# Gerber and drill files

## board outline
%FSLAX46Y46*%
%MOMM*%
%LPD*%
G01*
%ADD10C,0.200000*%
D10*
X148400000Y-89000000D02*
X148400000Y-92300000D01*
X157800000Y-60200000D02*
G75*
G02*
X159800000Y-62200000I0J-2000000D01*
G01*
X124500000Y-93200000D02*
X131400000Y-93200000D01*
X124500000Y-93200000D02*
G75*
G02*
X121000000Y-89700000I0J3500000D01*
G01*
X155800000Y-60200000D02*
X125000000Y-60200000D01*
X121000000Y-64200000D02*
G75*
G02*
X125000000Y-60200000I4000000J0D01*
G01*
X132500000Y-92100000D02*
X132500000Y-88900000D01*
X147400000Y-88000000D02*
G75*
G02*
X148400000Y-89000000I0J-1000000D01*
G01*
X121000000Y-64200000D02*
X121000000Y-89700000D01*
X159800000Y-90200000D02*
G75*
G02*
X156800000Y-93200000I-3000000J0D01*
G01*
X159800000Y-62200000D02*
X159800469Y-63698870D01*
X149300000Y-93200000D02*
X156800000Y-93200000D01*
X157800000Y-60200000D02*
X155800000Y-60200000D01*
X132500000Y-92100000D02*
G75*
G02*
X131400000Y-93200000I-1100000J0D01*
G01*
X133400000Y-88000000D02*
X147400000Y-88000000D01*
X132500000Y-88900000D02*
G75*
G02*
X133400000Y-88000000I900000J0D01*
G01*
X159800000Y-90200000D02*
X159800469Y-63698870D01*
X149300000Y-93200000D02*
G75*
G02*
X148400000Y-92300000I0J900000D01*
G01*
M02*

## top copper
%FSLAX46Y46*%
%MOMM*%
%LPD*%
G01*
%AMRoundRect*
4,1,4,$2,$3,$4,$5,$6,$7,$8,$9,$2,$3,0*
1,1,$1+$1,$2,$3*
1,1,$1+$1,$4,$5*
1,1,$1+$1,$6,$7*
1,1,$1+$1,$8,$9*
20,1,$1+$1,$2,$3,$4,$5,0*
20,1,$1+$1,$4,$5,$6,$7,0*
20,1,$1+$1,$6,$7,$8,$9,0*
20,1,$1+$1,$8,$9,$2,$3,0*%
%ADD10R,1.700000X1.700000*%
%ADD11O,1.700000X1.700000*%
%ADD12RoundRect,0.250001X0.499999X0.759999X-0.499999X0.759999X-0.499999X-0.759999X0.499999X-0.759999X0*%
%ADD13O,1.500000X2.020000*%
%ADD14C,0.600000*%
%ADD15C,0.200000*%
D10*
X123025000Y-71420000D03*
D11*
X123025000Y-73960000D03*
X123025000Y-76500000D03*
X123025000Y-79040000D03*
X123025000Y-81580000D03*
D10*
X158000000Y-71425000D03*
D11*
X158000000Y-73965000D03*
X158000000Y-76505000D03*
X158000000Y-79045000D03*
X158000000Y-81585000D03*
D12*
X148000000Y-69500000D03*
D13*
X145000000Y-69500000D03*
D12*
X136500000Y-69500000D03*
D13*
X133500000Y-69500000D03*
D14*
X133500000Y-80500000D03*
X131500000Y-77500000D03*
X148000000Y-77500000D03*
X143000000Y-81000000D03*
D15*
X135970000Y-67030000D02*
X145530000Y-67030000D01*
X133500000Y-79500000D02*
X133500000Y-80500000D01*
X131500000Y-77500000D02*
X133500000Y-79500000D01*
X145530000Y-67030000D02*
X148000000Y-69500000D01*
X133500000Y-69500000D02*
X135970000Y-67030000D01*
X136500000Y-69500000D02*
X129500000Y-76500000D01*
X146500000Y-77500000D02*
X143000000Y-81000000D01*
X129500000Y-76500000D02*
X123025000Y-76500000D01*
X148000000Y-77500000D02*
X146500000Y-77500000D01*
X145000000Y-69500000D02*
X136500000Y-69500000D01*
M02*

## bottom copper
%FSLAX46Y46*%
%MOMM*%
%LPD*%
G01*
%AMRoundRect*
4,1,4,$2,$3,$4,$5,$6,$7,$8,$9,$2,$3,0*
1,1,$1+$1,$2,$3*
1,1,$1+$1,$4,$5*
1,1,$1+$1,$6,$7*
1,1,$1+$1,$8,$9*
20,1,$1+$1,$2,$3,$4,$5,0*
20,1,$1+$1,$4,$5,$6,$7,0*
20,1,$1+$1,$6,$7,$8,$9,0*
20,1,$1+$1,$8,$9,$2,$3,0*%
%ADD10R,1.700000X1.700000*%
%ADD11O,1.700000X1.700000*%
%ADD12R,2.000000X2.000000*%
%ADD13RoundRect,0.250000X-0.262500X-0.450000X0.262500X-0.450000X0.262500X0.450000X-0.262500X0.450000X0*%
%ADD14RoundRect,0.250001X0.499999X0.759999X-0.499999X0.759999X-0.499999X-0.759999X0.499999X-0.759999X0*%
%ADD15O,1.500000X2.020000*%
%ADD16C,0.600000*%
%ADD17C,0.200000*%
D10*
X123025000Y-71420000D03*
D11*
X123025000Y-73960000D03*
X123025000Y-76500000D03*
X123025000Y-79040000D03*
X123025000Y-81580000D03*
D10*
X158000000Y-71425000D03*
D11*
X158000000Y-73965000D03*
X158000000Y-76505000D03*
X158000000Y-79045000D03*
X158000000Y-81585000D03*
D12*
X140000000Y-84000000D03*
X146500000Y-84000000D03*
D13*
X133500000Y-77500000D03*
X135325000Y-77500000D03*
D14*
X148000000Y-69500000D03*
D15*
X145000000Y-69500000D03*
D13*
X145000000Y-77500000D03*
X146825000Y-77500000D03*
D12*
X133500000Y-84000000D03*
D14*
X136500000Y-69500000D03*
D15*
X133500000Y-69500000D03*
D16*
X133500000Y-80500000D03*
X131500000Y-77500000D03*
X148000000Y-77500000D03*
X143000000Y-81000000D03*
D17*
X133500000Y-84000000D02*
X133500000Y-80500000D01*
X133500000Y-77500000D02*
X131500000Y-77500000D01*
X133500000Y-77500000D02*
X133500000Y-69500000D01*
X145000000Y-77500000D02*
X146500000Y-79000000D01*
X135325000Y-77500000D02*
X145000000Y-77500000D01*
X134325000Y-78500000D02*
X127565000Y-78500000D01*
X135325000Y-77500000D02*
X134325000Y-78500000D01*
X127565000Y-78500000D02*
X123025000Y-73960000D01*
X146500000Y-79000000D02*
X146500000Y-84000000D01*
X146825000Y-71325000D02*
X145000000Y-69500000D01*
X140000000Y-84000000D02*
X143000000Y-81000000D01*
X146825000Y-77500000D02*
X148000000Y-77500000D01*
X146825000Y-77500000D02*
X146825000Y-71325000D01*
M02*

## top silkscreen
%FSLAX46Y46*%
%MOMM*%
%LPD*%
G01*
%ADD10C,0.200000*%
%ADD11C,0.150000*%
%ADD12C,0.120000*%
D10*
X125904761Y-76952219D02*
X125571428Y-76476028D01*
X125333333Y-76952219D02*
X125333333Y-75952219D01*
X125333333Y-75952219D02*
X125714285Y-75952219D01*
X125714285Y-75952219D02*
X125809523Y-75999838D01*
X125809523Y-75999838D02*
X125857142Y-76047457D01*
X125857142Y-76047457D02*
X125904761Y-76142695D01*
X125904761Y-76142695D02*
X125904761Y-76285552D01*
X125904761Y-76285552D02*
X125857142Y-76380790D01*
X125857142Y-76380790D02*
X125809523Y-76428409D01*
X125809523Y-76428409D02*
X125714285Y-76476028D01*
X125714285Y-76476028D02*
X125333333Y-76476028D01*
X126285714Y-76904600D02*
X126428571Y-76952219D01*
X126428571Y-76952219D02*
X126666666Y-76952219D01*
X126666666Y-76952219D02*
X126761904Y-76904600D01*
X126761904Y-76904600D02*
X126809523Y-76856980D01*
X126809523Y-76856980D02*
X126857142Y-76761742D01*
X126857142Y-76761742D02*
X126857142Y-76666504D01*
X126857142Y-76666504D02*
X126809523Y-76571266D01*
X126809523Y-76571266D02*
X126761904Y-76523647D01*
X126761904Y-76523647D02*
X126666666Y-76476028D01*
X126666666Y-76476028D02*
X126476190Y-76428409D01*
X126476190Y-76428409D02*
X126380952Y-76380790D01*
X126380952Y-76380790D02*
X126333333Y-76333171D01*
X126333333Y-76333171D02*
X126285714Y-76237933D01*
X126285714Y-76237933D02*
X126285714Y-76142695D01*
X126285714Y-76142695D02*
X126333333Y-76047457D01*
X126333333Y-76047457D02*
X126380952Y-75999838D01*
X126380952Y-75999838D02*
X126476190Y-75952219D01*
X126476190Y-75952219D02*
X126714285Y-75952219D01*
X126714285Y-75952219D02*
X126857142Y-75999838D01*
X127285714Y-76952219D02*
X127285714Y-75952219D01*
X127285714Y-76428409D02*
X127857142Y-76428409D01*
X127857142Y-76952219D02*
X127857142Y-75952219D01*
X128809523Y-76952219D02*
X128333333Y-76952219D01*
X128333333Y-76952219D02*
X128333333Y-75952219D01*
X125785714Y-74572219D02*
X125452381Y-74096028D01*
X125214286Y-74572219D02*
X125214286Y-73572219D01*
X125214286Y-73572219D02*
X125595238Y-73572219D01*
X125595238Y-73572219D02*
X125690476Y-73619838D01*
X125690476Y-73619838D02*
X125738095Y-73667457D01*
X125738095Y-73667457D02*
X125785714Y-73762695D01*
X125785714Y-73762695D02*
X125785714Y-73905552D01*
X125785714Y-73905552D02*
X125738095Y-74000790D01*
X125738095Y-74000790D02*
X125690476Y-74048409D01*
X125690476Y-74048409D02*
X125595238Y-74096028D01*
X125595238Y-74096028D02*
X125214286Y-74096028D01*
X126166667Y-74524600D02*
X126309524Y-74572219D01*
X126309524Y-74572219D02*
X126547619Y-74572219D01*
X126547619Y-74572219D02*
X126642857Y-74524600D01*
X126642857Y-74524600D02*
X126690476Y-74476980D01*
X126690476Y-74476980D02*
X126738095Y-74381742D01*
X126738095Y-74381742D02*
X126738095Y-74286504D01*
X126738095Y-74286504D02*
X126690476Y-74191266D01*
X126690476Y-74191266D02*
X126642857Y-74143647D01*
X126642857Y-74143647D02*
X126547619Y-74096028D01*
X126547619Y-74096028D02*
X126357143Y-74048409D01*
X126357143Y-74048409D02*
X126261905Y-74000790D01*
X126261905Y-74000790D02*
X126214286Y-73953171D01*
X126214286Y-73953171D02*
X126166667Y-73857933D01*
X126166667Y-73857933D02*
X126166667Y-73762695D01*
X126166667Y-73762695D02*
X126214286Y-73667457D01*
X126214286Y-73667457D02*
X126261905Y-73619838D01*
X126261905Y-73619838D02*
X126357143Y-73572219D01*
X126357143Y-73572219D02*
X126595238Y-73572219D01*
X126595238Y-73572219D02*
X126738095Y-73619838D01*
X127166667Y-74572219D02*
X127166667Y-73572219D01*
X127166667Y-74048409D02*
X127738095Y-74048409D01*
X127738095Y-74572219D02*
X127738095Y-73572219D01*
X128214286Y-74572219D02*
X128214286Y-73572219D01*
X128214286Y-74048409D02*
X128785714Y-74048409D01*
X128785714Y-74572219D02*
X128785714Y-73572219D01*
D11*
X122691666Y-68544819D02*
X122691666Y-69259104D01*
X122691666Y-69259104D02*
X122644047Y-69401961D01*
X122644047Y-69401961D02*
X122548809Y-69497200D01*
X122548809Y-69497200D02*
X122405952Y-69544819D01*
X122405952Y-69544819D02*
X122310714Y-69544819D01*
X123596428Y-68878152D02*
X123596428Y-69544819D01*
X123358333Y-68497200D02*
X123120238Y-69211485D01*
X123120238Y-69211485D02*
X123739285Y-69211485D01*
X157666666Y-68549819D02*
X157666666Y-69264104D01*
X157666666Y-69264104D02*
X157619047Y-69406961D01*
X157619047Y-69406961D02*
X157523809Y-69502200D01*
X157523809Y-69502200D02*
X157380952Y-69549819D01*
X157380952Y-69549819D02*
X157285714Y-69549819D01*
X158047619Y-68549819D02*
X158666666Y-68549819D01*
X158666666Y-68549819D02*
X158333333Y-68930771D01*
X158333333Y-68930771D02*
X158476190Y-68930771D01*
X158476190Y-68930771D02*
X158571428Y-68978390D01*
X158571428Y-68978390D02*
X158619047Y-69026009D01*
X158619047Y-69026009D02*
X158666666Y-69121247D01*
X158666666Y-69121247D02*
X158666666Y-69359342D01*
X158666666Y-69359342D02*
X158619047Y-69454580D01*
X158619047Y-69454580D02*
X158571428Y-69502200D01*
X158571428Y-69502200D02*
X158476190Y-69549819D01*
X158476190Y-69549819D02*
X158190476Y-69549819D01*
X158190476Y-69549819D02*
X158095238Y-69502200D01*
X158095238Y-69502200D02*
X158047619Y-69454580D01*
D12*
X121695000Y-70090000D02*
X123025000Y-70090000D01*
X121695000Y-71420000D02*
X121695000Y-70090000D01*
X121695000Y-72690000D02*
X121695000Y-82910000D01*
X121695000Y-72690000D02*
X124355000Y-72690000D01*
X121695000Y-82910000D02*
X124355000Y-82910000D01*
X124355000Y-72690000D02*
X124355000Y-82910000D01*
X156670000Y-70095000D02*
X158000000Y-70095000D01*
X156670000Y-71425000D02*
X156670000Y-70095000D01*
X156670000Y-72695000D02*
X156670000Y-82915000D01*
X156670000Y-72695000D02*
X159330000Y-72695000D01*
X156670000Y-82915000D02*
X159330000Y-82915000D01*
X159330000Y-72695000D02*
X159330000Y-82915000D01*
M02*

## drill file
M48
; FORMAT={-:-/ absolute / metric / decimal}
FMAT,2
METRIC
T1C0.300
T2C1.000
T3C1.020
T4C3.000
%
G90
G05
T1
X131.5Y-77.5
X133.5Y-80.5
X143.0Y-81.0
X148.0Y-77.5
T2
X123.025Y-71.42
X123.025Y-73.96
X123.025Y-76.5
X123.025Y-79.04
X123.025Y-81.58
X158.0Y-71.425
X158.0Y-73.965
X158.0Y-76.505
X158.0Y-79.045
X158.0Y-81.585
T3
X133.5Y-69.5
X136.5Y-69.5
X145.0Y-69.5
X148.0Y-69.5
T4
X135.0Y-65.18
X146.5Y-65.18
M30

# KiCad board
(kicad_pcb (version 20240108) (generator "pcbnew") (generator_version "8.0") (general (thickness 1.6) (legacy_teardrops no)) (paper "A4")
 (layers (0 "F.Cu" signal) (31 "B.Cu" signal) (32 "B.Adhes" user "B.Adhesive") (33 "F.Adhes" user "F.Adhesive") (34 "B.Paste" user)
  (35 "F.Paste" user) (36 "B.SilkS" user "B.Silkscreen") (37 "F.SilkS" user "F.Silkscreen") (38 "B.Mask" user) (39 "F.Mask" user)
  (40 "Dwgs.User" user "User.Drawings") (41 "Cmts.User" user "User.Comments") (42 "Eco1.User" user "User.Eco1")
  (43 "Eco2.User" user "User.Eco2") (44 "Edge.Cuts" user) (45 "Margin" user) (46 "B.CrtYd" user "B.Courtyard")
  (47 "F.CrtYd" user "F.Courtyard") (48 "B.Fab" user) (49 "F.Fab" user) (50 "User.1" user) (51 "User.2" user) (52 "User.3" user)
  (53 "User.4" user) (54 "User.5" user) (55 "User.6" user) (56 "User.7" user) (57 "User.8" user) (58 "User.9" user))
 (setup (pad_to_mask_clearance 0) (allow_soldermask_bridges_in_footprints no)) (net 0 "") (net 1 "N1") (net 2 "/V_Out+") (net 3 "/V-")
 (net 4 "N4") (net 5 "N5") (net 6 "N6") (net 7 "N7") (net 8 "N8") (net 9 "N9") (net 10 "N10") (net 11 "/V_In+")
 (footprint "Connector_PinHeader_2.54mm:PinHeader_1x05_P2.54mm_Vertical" (layer "F.Cu") (at 123.025 71.42)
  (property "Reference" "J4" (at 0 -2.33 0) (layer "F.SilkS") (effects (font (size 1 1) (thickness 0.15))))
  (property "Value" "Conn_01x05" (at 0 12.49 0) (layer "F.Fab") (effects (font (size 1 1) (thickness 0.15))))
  (fp_line (start -1.33 -1.33) (end 0 -1.33) (stroke (width 0.12) (type solid)) (layer "F.SilkS"))
  (fp_line (start -1.33 0) (end -1.33 -1.33) (stroke (width 0.12) (type solid)) (layer "F.SilkS"))
  (fp_line (start -1.33 1.27) (end -1.33 11.49) (stroke (width 0.12) (type solid)) (layer "F.SilkS"))
  (fp_line (start -1.33 1.27) (end 1.33 1.27) (stroke (width 0.12) (type solid)) (layer "F.SilkS"))
  (fp_line (start -1.33 11.49) (end 1.33 11.49) (stroke (width 0.12) (type solid)) (layer "F.SilkS"))
  (fp_line (start 1.33 1.27) (end 1.33 11.49) (stroke (width 0.12) (type solid)) (layer "F.SilkS"))
  (pad "1" thru_hole rect (at 0 0) (size 1.7 1.7) (drill 1) (layers "*.Cu" "*.Mask") (remove_unused_layers no) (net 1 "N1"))
  (pad "2" thru_hole oval (at 0 2.54) (size 1.7 1.7) (drill 1) (layers "*.Cu" "*.Mask") (remove_unused_layers no) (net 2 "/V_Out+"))
  (pad "3" thru_hole oval (at 0 5.08) (size 1.7 1.7) (drill 1) (layers "*.Cu" "*.Mask") (remove_unused_layers no) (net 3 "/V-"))
  (pad "4" thru_hole oval (at 0 7.62) (size 1.7 1.7) (drill 1) (layers "*.Cu" "*.Mask") (remove_unused_layers no) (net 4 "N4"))
  (pad "5" thru_hole oval (at 0 10.16) (size 1.7 1.7) (drill 1) (layers "*.Cu" "*.Mask") (remove_unused_layers no) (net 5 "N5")))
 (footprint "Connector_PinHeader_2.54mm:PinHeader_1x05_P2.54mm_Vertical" (layer "F.Cu") (at 158 71.425)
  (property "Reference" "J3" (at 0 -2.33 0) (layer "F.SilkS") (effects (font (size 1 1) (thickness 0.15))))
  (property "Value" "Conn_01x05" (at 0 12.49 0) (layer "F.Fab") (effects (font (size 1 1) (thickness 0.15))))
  (fp_line (start -1.33 -1.33) (end 0 -1.33) (stroke (width 0.12) (type solid)) (layer "F.SilkS"))
  (fp_line (start -1.33 0) (end -1.33 -1.33) (stroke (width 0.12) (type solid)) (layer "F.SilkS"))
  (fp_line (start -1.33 1.27) (end -1.33 11.49) (stroke (width 0.12) (type solid)) (layer "F.SilkS"))
  (fp_line (start -1.33 1.27) (end 1.33 1.27) (stroke (width 0.12) (type solid)) (layer "F.SilkS"))
  (fp_line (start -1.33 11.49) (end 1.33 11.49) (stroke (width 0.12) (type solid)) (layer "F.SilkS"))
  (fp_line (start 1.33 1.27) (end 1.33 11.49) (stroke (width 0.12) (type solid)) (layer "F.SilkS"))
  (pad "1" thru_hole rect (at 0 0) (size 1.7 1.7) (drill 1) (layers "*.Cu" "*.Mask") (remove_unused_layers no) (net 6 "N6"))
  (pad "2" thru_hole oval (at 0 2.54) (size 1.7 1.7) (drill 1) (layers "*.Cu" "*.Mask") (remove_unused_layers no) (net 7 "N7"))
  (pad "3" thru_hole oval (at 0 5.08) (size 1.7 1.7) (drill 1) (layers "*.Cu" "*.Mask") (remove_unused_layers no) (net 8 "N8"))
  (pad "4" thru_hole oval (at 0 7.62) (size 1.7 1.7) (drill 1) (layers "*.Cu" "*.Mask") (remove_unused_layers no) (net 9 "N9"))
  (pad "5" thru_hole oval (at 0 10.16) (size 1.7 1.7) (drill 1) (layers "*.Cu" "*.Mask") (remove_unused_layers no) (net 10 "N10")))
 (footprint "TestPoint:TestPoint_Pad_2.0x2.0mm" (layer "B.Cu") (at 140 84 180)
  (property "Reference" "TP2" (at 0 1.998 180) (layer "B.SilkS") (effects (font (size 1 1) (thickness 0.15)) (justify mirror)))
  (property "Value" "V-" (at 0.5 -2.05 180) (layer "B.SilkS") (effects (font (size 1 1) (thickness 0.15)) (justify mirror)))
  (pad "1" smd rect (at 0 0 180) (size 2 2) (layers "B.Cu" "B.Mask") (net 3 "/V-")))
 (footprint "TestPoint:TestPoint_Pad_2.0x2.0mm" (layer "B.Cu") (at 146.5 84 180)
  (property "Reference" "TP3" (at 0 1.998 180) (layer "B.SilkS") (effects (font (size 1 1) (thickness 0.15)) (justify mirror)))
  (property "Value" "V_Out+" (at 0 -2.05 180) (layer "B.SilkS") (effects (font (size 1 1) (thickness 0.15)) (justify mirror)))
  (pad "1" smd rect (at 0 0 180) (size 2 2) (layers "B.Cu" "B.Mask") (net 2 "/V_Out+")))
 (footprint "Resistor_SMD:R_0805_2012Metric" (layer "B.Cu") (at 134.4125 77.5)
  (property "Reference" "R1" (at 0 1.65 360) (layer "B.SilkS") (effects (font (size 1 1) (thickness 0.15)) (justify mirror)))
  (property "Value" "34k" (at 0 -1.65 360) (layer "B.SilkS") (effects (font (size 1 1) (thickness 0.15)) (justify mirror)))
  (pad "1" smd roundrect (at -0.9125 0) (size 1.025 1.4) (layers "B.Cu" "B.Paste" "B.Mask") (roundrect_rratio 0.243902) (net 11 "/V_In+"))
  (pad "2" smd roundrect (at 0.9125 0) (size 1.025 1.4) (layers "B.Cu" "B.Paste" "B.Mask") (roundrect_rratio 0.243902) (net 2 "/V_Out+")))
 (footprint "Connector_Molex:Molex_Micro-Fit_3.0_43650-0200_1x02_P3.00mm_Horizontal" (layer "B.Cu") (at 148 69.5 180)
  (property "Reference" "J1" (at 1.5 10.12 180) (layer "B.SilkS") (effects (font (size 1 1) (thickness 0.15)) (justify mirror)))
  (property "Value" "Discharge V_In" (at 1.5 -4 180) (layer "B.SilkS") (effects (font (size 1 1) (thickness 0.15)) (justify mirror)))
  (pad "" np_thru_hole circle (at 1.5 4.32 180) (size 3 3) (drill 3) (layers "*.Cu" "*.Mask"))
  (pad "1" thru_hole roundrect (at 0 0 180) (size 1.5 2.02) (drill 1.02) (layers "*.Cu" "*.Mask") (remove_unused_layers no)
   (roundrect_rratio 0.166667) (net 11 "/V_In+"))
  (pad "2" thru_hole oval (at 3 0 180) (size 1.5 2.02) (drill 1.02) (layers "*.Cu" "*.Mask") (remove_unused_layers no) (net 3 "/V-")))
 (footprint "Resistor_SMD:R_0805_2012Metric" (layer "B.Cu") (at 145.9125 77.5)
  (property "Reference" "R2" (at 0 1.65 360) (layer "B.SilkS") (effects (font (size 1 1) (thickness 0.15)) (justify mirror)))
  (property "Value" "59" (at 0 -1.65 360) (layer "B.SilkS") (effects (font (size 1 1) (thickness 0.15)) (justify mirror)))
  (pad "1" smd roundrect (at -0.9125 0) (size 1.025 1.4) (layers "B.Cu" "B.Paste" "B.Mask") (roundrect_rratio 0.243902) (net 2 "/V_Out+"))
  (pad "2" smd roundrect (at 0.9125 0) (size 1.025 1.4) (layers "B.Cu" "B.Paste" "B.Mask") (roundrect_rratio 0.243902) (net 3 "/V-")))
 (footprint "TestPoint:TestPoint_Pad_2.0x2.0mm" (layer "B.Cu") (at 133.5 84 180)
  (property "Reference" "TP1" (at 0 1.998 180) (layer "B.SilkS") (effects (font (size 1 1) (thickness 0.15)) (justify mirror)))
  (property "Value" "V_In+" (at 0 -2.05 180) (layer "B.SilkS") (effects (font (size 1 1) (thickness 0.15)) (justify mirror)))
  (pad "1" smd rect (at 0 0 180) (size 2 2) (layers "B.Cu" "B.Mask") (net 11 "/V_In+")))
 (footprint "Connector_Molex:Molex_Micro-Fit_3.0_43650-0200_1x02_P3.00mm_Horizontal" (layer "B.Cu") (at 136.5 69.5 180)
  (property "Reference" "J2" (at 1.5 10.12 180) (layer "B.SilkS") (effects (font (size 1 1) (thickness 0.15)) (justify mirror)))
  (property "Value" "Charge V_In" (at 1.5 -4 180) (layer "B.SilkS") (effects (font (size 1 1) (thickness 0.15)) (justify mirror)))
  (pad "" np_thru_hole circle (at 1.5 4.32 180) (size 3 3) (drill 3) (layers "*.Cu" "*.Mask"))
  (pad "1" thru_hole roundrect (at 0 0 180) (size 1.5 2.02) (drill 1.02) (layers "*.Cu" "*.Mask") (remove_unused_layers no)
   (roundrect_rratio 0.166667) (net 3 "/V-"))
  (pad "2" thru_hole oval (at 3 0 180) (size 1.5 2.02) (drill 1.02) (layers "*.Cu" "*.Mask") (remove_unused_layers no) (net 11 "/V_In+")))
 (gr_line (start 148.4 89) (end 148.4 92.3) (stroke (width 0.2) (type solid)) (layer "Edge.Cuts"))
 (gr_arc (start 157.8 60.2) (mid 159.214214 60.785786) (end 159.8 62.2) (stroke (width 0.2) (type solid)) (layer "Edge.Cuts"))
 (gr_line (start 124.5 93.2) (end 131.4 93.2) (stroke (width 0.2) (type solid)) (layer "Edge.Cuts"))
 (gr_arc (start 124.5 93.2) (mid 122.025126 92.174874) (end 121 89.7) (stroke (width 0.2) (type solid)) (layer "Edge.Cuts"))
 (gr_line (start 155.8 60.2) (end 125 60.2) (stroke (width 0.2) (type solid)) (layer "Edge.Cuts"))
 (gr_arc (start 121 64.2) (mid 122.171573 61.371573) (end 125 60.2) (stroke (width 0.2) (type solid)) (layer "Edge.Cuts"))
 (gr_line (start 132.5 92.1) (end 132.5 88.9) (stroke (width 0.2) (type solid)) (layer "Edge.Cuts"))
 (gr_arc (start 147.4 88) (mid 148.107107 88.292893) (end 148.4 89) (stroke (width 0.2) (type solid)) (layer "Edge.Cuts"))
 (gr_line (start 121 64.2) (end 121 89.7) (stroke (width 0.2) (type solid)) (layer "Edge.Cuts"))
 (gr_arc (start 159.8 90.2) (mid 158.92132 92.32132) (end 156.8 93.2) (stroke (width 0.2) (type solid)) (layer "Edge.Cuts"))
 (gr_line (start 159.8 62.2) (end 159.800469 63.69887) (stroke (width 0.2) (type solid)) (layer "Edge.Cuts"))
 (gr_line (start 149.3 93.2) (end 156.8 93.2) (stroke (width 0.2) (type solid)) (layer "Edge.Cuts"))
 (gr_line (start 157.8 60.2) (end 155.8 60.2) (stroke (width 0.2) (type solid)) (layer "Edge.Cuts"))
 (gr_arc (start 132.5 92.1) (mid 132.177817 92.877817) (end 131.4 93.2) (stroke (width 0.2) (type solid)) (layer "Edge.Cuts"))
 (gr_line (start 133.4 88) (end 147.4 88) (stroke (width 0.2) (type solid)) (layer "Edge.Cuts"))
 (gr_arc (start 132.5 88.9) (mid 132.763604 88.263604) (end 133.4 88) (stroke (width 0.2) (type solid)) (layer "Edge.Cuts"))
 (gr_line (start 159.8 90.2) (end 159.800469 63.69887) (stroke (width 0.2) (type solid)) (layer "Edge.Cuts"))
 (gr_arc (start 149.3 93.2) (mid 148.663604 92.936396) (end 148.4 92.3) (stroke (width 0.2) (type solid)) (layer "Edge.Cuts"))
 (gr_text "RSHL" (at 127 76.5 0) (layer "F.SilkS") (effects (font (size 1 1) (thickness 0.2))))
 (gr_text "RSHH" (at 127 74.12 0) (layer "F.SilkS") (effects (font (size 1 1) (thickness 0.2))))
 (segment (start 135.97 67.03) (end 145.53 67.03) (width 0.2) (layer "F.Cu") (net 11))
 (segment (start 133.5 79.5) (end 133.5 80.5) (width 0.2) (layer "F.Cu") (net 11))
 (segment (start 131.5 77.5) (end 133.5 79.5) (width 0.2) (layer "F.Cu") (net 11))
 (segment (start 145.53 67.03) (end 148 69.5) (width 0.2) (layer "F.Cu") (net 11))
 (segment (start 133.5 69.5) (end 135.97 67.03) (width 0.2) (layer "F.Cu") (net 11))
 (via (at 133.5 80.5) (size 0.6) (drill 0.3) (layers "F.Cu" "B.Cu") (free yes) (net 11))
 (via (at 131.5 77.5) (size 0.6) (drill 0.3) (layers "F.Cu" "B.Cu") (free yes) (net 11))
 (segment (start 133.5 84) (end 133.5 80.5) (width 0.2) (layer "B.Cu") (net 11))
 (segment (start 133.5 77.5) (end 131.5 77.5) (width 0.2) (layer "B.Cu") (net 11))
 (segment (start 133.5 77.5) (end 133.5 69.5) (width 0.2) (layer "B.Cu") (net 11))
 (segment (start 145 77.5) (end 146.5 79) (width 0.2) (layer "B.Cu") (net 2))
 (segment (start 135.325 77.5) (end 145 77.5) (width 0.2) (layer "B.Cu") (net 2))
 (segment (start 134.325 78.5) (end 127.565 78.5) (width 0.2) (layer "B.Cu") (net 2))
 (segment (start 135.325 77.5) (end 134.325 78.5) (width 0.2) (layer "B.Cu") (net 2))
 (segment (start 127.565 78.5) (end 123.025 73.96) (width 0.2) (layer "B.Cu") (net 2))
 (segment (start 146.5 79) (end 146.5 84) (width 0.2) (layer "B.Cu") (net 2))
 (segment (start 136.5 69.5) (end 129.5 76.5) (width 0.2) (layer "F.Cu") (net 3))
 (segment (start 146.5 77.5) (end 143 81) (width 0.2) (layer "F.Cu") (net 3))
 (segment (start 129.5 76.5) (end 123.025 76.5) (width 0.2) (layer "F.Cu") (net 3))
 (segment (start 148 77.5) (end 146.5 77.5) (width 0.2) (layer "F.Cu") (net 3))
 (segment (start 145 69.5) (end 136.5 69.5) (width 0.2) (layer "F.Cu") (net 3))
 (via (at 148 77.5) (size 0.6) (drill 0.3) (layers "F.Cu" "B.Cu") (free yes) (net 3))
 (via (at 143 81) (size 0.6) (drill 0.3) (layers "F.Cu" "B.Cu") (free yes) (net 3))
 (segment (start 146.825 71.325) (end 145 69.5) (width 0.2) (layer "B.Cu") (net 3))
 (segment (start 140 84) (end 143 81) (width 0.2) (layer "B.Cu") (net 3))
 (segment (start 146.825 77.5) (end 148 77.5) (width 0.2) (layer "B.Cu") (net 3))
 (segment (start 146.825 77.5) (end 146.825 71.325) (width 0.2) (layer "B.Cu") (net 3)))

